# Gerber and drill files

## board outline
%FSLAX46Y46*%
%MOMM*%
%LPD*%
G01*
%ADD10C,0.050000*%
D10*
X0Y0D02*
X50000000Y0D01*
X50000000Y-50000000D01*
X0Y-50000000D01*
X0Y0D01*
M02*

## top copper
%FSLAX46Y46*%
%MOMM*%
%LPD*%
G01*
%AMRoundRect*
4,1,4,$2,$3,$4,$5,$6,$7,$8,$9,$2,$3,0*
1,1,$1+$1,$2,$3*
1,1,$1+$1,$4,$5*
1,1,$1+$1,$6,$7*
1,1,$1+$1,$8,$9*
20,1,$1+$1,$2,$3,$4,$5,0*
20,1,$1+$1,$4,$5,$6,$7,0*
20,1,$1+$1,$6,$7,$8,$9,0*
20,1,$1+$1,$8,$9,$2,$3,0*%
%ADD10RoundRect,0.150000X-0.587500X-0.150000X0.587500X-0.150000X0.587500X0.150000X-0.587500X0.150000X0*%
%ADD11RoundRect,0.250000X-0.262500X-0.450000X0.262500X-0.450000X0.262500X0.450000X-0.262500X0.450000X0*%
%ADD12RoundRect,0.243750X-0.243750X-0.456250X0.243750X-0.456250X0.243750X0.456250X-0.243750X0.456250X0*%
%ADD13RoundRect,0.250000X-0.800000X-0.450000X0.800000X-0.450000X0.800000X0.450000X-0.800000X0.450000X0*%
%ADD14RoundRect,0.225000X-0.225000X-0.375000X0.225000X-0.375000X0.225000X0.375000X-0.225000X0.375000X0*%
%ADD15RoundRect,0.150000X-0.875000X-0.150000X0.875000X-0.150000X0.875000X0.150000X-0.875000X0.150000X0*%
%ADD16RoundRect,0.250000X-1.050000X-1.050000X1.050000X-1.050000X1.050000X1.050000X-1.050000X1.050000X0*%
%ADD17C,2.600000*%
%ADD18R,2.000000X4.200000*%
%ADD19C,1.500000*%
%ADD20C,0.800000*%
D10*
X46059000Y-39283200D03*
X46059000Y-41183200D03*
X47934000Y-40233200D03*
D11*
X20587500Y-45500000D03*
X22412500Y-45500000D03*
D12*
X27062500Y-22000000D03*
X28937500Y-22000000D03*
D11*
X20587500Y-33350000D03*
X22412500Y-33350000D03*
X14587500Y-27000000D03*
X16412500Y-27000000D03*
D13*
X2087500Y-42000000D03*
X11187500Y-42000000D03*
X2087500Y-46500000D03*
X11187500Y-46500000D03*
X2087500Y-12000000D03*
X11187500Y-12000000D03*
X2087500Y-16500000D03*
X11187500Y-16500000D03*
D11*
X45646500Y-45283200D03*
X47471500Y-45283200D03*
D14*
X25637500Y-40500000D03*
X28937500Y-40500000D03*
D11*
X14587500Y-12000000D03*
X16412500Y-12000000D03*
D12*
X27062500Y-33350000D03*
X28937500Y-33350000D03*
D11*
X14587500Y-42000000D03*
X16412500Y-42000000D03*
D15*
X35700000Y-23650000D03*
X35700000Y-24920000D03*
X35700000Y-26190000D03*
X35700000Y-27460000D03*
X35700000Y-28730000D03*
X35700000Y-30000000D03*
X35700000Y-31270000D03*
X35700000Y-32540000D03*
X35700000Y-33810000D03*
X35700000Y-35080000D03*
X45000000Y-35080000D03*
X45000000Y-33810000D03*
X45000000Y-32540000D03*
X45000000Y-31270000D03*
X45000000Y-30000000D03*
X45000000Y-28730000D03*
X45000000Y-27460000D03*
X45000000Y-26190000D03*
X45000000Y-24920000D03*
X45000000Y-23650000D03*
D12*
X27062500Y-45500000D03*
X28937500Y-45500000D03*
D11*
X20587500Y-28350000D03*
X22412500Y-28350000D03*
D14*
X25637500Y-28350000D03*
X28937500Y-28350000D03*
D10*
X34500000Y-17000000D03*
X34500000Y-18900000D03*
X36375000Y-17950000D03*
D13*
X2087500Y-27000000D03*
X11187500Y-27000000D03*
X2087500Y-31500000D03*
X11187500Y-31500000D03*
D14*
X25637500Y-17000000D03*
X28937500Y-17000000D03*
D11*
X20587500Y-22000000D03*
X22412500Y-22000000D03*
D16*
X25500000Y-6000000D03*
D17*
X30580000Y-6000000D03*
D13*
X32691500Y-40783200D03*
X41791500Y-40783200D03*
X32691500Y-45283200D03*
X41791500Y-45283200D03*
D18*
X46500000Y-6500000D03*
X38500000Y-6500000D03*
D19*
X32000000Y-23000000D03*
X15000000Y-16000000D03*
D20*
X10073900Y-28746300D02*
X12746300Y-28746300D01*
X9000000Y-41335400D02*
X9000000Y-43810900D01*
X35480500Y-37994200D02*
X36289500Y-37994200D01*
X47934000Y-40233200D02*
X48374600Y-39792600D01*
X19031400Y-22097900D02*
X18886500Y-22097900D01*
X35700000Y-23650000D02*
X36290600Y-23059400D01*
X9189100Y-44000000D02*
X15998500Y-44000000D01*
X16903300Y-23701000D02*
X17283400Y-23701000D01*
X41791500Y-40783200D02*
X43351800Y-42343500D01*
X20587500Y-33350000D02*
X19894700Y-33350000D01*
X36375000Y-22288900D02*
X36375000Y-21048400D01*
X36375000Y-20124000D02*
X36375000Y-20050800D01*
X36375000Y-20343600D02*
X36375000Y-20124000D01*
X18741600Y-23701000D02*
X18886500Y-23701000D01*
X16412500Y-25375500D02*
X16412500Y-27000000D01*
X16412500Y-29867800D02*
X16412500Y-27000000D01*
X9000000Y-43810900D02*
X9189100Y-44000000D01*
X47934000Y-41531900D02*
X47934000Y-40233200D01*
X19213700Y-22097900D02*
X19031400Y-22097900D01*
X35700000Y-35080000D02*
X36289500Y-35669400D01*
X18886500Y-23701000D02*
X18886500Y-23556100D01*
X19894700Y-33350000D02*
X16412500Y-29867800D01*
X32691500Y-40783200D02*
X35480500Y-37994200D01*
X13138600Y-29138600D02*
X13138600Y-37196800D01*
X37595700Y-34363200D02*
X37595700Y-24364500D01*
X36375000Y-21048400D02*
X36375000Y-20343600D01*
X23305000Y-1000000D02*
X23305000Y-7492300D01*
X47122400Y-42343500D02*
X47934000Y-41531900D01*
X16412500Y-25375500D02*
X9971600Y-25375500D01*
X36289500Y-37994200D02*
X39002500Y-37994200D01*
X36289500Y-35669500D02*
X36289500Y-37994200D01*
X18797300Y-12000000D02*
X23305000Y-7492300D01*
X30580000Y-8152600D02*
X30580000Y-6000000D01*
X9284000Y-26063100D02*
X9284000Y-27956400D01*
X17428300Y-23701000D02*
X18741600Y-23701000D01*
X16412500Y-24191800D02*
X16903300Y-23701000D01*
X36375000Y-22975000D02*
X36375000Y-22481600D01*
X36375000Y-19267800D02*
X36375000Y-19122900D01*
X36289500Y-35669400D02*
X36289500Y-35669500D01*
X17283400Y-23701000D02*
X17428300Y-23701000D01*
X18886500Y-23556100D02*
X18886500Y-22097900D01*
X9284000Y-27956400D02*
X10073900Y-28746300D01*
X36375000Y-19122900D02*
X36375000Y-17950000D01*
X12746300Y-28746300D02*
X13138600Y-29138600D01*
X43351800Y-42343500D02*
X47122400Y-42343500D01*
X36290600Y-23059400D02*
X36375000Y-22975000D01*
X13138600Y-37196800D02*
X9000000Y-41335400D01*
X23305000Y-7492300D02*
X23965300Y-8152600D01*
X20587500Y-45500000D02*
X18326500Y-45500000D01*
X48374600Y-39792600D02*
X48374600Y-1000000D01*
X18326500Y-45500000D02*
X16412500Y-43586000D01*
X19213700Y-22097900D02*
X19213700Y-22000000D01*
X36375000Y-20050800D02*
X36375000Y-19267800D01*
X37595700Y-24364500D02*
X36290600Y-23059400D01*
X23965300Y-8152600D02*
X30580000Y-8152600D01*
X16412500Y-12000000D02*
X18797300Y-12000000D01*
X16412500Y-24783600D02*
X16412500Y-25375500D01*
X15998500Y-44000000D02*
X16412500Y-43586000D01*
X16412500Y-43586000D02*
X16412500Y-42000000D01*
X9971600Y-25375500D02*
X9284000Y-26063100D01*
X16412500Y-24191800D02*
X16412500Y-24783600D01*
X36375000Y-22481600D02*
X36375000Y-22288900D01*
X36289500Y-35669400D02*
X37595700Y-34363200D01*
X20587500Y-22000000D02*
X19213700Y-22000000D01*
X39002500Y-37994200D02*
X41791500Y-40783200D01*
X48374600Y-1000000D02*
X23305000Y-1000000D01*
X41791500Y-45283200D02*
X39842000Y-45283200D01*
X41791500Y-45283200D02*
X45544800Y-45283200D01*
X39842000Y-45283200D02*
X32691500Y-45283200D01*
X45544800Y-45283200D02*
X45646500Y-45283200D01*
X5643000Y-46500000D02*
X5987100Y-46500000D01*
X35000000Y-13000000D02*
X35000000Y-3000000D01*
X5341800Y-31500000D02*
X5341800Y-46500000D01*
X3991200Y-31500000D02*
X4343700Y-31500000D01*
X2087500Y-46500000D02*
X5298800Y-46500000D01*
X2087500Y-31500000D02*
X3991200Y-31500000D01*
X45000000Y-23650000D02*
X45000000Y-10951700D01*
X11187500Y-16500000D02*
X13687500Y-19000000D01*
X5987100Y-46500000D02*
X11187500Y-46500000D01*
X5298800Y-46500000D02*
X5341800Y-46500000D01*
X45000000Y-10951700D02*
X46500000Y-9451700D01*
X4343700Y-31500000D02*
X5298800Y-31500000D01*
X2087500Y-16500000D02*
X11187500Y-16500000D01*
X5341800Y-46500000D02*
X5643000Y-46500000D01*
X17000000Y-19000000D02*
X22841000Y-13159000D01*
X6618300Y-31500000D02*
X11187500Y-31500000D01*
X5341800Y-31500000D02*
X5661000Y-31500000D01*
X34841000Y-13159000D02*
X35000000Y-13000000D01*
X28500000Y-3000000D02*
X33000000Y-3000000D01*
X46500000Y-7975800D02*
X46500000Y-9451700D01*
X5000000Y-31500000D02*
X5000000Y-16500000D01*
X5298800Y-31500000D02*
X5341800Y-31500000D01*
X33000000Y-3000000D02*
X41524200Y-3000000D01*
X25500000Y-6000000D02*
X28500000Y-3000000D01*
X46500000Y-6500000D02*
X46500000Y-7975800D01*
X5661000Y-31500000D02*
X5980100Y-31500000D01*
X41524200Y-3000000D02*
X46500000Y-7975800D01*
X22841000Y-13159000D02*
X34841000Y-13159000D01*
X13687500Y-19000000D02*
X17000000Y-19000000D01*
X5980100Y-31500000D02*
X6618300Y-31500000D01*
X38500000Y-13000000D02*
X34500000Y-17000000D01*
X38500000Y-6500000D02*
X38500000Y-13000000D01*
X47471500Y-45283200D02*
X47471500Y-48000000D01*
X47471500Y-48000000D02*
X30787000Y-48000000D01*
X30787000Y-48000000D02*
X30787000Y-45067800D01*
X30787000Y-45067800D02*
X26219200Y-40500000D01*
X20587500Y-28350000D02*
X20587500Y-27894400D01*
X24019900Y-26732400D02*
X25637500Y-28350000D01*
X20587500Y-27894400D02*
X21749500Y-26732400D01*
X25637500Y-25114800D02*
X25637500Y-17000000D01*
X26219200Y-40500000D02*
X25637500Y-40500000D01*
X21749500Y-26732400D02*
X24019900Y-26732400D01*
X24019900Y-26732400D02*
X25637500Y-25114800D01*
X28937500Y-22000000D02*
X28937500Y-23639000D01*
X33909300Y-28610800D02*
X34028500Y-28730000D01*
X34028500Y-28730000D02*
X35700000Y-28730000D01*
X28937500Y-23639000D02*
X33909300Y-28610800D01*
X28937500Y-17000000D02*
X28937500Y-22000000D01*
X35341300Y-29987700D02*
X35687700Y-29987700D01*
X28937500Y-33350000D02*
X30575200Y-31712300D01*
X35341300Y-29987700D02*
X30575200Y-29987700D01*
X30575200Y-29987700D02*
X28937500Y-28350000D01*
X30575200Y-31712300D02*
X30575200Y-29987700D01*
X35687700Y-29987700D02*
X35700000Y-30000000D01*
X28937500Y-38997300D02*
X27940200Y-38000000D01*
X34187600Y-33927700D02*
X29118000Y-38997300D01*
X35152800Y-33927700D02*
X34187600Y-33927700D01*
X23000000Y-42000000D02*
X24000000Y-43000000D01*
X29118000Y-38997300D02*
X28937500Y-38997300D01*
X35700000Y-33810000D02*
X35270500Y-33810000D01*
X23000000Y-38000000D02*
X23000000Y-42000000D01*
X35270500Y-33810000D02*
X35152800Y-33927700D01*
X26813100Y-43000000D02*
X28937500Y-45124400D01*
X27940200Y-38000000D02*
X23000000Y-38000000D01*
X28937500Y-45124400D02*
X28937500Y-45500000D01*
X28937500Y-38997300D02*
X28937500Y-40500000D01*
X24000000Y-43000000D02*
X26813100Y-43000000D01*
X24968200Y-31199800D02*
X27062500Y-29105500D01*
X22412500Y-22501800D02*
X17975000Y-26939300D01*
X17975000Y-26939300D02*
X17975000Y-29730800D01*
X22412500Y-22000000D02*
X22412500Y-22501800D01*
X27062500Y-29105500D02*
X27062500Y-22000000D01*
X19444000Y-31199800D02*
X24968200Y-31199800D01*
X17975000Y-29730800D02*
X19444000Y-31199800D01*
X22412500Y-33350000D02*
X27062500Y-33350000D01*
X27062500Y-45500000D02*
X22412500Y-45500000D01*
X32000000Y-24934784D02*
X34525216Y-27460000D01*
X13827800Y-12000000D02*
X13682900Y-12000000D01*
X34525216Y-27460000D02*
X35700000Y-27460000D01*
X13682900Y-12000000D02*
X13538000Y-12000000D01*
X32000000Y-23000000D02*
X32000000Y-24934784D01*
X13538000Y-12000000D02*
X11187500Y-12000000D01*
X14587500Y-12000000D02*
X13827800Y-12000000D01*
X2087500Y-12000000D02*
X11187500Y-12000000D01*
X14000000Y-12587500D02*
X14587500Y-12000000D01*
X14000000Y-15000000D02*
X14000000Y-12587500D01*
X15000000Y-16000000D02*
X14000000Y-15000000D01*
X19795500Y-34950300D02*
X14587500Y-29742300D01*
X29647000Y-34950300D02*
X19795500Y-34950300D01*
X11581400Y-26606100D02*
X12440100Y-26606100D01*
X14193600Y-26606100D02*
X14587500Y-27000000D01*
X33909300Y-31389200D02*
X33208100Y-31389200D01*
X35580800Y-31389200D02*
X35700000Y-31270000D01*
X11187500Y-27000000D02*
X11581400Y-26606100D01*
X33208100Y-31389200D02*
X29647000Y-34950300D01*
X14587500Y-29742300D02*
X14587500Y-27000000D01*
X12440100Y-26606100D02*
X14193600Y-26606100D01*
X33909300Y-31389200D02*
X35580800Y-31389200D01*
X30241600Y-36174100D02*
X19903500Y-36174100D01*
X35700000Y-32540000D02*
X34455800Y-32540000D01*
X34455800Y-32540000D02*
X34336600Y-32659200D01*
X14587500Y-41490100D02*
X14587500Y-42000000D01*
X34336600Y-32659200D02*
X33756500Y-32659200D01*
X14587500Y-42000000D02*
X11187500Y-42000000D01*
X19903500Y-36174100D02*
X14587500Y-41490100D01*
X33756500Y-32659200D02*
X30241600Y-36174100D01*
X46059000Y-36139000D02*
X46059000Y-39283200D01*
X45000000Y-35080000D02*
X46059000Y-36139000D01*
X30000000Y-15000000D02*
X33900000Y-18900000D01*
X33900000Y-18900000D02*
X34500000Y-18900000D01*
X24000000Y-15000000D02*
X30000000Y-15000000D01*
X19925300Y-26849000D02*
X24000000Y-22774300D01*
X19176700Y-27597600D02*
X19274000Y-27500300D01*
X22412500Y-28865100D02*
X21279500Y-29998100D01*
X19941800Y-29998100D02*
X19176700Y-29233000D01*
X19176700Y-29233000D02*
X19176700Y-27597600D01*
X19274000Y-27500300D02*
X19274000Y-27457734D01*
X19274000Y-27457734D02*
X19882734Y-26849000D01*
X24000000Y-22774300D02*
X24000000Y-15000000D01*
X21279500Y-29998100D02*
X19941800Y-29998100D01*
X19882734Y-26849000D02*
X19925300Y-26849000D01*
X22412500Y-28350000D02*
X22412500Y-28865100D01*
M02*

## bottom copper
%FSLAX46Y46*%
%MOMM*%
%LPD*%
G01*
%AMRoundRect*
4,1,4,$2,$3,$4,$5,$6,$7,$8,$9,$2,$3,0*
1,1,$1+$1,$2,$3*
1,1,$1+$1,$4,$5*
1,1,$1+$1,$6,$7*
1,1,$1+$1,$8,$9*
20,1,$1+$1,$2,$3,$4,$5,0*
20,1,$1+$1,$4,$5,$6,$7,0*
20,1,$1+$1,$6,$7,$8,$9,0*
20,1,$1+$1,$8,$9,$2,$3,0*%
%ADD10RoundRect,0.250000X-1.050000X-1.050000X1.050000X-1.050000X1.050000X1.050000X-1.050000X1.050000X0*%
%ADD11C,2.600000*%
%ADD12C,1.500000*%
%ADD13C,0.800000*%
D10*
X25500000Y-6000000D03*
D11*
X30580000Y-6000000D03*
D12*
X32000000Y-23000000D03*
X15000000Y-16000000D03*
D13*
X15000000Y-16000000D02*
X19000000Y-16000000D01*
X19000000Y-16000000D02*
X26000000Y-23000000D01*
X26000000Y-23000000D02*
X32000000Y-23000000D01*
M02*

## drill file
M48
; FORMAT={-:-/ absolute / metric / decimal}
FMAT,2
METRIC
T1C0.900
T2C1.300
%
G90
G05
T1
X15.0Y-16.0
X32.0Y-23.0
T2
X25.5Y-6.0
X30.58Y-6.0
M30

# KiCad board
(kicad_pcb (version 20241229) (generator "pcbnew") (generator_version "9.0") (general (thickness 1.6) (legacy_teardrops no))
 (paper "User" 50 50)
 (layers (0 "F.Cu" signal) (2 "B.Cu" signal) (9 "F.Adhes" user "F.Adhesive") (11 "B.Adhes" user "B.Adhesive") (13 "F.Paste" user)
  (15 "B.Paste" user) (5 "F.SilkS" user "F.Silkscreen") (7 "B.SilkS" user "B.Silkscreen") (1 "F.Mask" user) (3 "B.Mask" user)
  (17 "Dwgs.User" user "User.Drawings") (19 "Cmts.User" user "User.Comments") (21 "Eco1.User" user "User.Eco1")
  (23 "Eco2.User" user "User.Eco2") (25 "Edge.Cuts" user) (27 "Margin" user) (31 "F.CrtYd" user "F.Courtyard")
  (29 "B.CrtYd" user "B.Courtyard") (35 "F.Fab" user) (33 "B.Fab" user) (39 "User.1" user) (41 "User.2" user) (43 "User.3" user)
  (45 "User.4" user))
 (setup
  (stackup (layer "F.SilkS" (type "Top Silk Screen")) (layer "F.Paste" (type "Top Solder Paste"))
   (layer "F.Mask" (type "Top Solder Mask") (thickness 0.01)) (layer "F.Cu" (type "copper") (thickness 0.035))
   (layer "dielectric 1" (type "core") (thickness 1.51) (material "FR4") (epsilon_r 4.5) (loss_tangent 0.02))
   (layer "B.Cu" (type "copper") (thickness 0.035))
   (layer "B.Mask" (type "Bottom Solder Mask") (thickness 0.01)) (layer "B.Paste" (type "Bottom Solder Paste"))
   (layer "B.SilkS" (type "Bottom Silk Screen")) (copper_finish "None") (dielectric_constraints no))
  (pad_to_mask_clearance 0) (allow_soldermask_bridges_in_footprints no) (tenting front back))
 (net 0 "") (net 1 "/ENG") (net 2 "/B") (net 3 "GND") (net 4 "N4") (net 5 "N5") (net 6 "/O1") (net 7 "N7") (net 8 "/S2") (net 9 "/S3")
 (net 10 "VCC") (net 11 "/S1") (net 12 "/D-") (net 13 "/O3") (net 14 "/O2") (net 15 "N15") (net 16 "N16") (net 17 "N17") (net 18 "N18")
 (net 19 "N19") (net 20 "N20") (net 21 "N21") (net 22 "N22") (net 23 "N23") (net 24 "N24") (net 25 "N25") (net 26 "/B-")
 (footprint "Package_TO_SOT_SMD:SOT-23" (layer "F.Cu") (at 46.9965 40.2332)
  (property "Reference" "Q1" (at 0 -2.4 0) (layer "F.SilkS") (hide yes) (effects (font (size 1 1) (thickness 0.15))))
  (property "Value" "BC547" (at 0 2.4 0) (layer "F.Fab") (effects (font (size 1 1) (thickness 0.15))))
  (pad "1" smd roundrect (at -0.9375 -0.95) (size 1.475 0.6) (layers "F.Cu" "F.Mask" "F.Paste") (roundrect_rratio 0.25) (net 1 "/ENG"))
  (pad "2" smd roundrect (at -0.9375 0.95) (size 1.475 0.6) (layers "F.Cu" "F.Mask" "F.Paste") (roundrect_rratio 0.25) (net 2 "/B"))
  (pad "3" smd roundrect (at 0.9375 0) (size 1.475 0.6) (layers "F.Cu" "F.Mask" "F.Paste") (roundrect_rratio 0.25) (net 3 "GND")))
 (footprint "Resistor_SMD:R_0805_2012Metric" (layer "F.Cu") (at 21.5 45.5)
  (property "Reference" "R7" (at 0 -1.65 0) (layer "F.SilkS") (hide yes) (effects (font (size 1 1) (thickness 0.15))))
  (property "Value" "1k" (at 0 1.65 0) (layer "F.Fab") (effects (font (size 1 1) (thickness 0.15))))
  (pad "1" smd roundrect (at -0.9125 0) (size 1.025 1.4) (layers "F.Cu" "F.Mask" "F.Paste") (roundrect_rratio 0.243902) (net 3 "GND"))
  (pad "2" smd roundrect (at 0.9125 0) (size 1.025 1.4) (layers "F.Cu" "F.Mask" "F.Paste") (roundrect_rratio 0.243902) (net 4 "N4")))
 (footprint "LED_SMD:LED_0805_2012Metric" (layer "F.Cu") (at 28 22)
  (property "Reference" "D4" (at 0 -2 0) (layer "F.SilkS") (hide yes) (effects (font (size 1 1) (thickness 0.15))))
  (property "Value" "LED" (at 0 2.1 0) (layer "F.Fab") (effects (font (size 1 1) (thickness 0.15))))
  (pad "1" smd roundrect (at -0.9375 0) (size 0.975 1.4) (layers "F.Cu" "F.Mask" "F.Paste") (roundrect_rratio 0.25) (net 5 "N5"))
  (pad "2" smd roundrect (at 0.9375 0) (size 0.975 1.4) (layers "F.Cu" "F.Mask" "F.Paste") (roundrect_rratio 0.25) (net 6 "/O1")))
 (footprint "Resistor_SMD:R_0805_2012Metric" (layer "F.Cu") (at 21.5 33.35)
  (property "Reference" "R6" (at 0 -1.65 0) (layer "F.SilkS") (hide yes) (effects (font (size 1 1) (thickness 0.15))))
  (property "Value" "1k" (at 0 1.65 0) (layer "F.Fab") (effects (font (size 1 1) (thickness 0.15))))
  (pad "1" smd roundrect (at -0.9125 0) (size 1.025 1.4) (layers "F.Cu" "F.Mask" "F.Paste") (roundrect_rratio 0.243902) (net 3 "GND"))
  (pad "2" smd roundrect (at 0.9125 0) (size 1.025 1.4) (layers "F.Cu" "F.Mask" "F.Paste") (roundrect_rratio 0.243902) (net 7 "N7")))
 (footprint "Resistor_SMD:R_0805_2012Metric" (layer "F.Cu") (at 15.5 27)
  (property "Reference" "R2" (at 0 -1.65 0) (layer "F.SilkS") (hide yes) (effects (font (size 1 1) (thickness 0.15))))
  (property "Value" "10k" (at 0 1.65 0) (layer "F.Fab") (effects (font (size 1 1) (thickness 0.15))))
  (pad "1" smd roundrect (at -0.9125 0) (size 1.025 1.4) (layers "F.Cu" "F.Mask" "F.Paste") (roundrect_rratio 0.243902) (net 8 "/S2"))
  (pad "2" smd roundrect (at 0.9125 0) (size 1.025 1.4) (layers "F.Cu" "F.Mask" "F.Paste") (roundrect_rratio 0.243902) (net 3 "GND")))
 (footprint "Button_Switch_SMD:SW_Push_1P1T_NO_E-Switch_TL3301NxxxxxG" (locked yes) (layer "F.Cu") (at 6.6375 44.25)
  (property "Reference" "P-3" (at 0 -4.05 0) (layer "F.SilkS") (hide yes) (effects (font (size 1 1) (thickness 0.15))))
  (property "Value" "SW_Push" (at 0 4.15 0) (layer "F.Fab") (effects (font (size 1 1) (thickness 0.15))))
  (pad "1" smd roundrect (at -4.55 -2.25) (size 2.1 1.4) (layers "F.Cu" "F.Mask" "F.Paste") (roundrect_rratio 0.1785714286) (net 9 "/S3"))
  (pad "1" smd roundrect (at 4.55 -2.25) (size 2.1 1.4) (layers "F.Cu" "F.Mask" "F.Paste") (roundrect_rratio 0.1785714286) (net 9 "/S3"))
  (pad "2" smd roundrect (at -4.55 2.25) (size 2.1 1.4) (layers "F.Cu" "F.Mask" "F.Paste") (roundrect_rratio 0.1785714286) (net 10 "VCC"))
  (pad "2" smd roundrect (at 4.55 2.25) (size 2.1 1.4) (layers "F.Cu" "F.Mask" "F.Paste") (roundrect_rratio 0.1785714286) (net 10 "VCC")))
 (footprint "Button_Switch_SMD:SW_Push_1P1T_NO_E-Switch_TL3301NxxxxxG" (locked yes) (layer "F.Cu") (at 6.6375 14.25)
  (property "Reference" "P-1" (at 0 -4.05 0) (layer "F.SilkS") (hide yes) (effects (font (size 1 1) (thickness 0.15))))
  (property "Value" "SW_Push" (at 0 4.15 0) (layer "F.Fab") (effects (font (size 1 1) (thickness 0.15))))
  (pad "1" smd roundrect (at -4.55 -2.25) (size 2.1 1.4) (layers "F.Cu" "F.Mask" "F.Paste") (roundrect_rratio 0.1785714286) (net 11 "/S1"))
  (pad "1" smd roundrect (at 4.55 -2.25) (size 2.1 1.4) (layers "F.Cu" "F.Mask" "F.Paste") (roundrect_rratio 0.1785714286) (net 11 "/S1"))
  (pad "2" smd roundrect (at -4.55 2.25) (size 2.1 1.4) (layers "F.Cu" "F.Mask" "F.Paste") (roundrect_rratio 0.1785714286) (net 10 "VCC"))
  (pad "2" smd roundrect (at 4.55 2.25) (size 2.1 1.4) (layers "F.Cu" "F.Mask" "F.Paste") (roundrect_rratio 0.1785714286) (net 10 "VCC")))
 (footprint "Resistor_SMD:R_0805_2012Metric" (layer "F.Cu") (at 46.559 45.2832)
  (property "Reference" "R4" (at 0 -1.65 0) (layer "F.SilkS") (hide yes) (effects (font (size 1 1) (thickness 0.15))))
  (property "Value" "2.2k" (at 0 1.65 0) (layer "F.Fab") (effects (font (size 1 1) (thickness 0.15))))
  (pad "1" smd roundrect (at -0.9125 0) (size 1.025 1.4) (layers "F.Cu" "F.Mask" "F.Paste") (roundrect_rratio 0.243902) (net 2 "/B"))
  (pad "2" smd roundrect (at 0.9125 0) (size 1.025 1.4) (layers "F.Cu" "F.Mask" "F.Paste") (roundrect_rratio 0.243902) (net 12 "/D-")))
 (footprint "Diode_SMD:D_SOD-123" (layer "F.Cu") (at 27.2875 40.5)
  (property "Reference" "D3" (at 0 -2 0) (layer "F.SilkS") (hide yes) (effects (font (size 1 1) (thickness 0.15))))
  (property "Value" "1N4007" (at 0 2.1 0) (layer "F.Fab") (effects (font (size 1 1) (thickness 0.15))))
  (pad "1" smd roundrect (at -1.65 0) (size 0.9 1.2) (layers "F.Cu" "F.Mask" "F.Paste") (roundrect_rratio 0.25) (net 12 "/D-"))
  (pad "2" smd roundrect (at 1.65 0) (size 0.9 1.2) (layers "F.Cu" "F.Mask" "F.Paste") (roundrect_rratio 0.25) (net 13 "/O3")))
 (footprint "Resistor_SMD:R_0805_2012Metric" (layer "F.Cu") (at 15.5 12)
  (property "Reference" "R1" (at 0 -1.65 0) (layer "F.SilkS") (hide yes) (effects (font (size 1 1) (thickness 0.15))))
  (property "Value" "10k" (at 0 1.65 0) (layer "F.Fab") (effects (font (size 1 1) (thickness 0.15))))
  (pad "1" smd roundrect (at -0.9125 0) (size 1.025 1.4) (layers "F.Cu" "F.Mask" "F.Paste") (roundrect_rratio 0.243902) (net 11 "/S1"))
  (pad "2" smd roundrect (at 0.9125 0) (size 1.025 1.4) (layers "F.Cu" "F.Mask" "F.Paste") (roundrect_rratio 0.243902) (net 3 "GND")))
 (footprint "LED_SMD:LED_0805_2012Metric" (layer "F.Cu") (at 28 33.35)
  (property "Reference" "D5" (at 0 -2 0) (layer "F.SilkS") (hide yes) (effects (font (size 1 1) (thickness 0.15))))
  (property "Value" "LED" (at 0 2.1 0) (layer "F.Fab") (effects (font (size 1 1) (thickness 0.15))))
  (pad "1" smd roundrect (at -0.9375 0) (size 0.975 1.4) (layers "F.Cu" "F.Mask" "F.Paste") (roundrect_rratio 0.25) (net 7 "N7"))
  (pad "2" smd roundrect (at 0.9375 0) (size 0.975 1.4) (layers "F.Cu" "F.Mask" "F.Paste") (roundrect_rratio 0.25) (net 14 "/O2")))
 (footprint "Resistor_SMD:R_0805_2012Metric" (layer "F.Cu") (at 15.5 42)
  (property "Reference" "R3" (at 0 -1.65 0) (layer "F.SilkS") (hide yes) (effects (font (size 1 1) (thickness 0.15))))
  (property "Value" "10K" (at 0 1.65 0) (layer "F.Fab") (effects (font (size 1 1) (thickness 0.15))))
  (pad "1" smd roundrect (at -0.9125 0) (size 1.025 1.4) (layers "F.Cu" "F.Mask" "F.Paste") (roundrect_rratio 0.243902) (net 9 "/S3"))
  (pad "2" smd roundrect (at 0.9125 0) (size 1.025 1.4) (layers "F.Cu" "F.Mask" "F.Paste") (roundrect_rratio 0.243902) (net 3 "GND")))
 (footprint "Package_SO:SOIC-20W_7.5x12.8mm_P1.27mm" (layer "F.Cu") (at 40.35 29.365)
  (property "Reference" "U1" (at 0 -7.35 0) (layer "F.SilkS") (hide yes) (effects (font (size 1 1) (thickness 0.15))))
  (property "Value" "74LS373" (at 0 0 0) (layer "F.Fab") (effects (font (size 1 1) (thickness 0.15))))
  (pad "1" smd roundrect (at -4.65 -5.715) (size 2.05 0.6) (layers "F.Cu" "F.Mask" "F.Paste") (roundrect_rratio 0.25) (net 3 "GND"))
  (pad "2" smd roundrect (at -4.65 -4.445) (size 2.05 0.6) (layers "F.Cu" "F.Mask" "F.Paste") (roundrect_rratio 0.25) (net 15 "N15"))
  (pad "3" smd roundrect (at -4.65 -3.175) (size 2.05 0.6) (layers "F.Cu" "F.Mask" "F.Paste") (roundrect_rratio 0.25) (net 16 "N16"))
  (pad "4" smd roundrect (at -4.65 -1.905) (size 2.05 0.6) (layers "F.Cu" "F.Mask" "F.Paste") (roundrect_rratio 0.25) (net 11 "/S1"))
  (pad "5" smd roundrect (at -4.65 -0.635) (size 2.05 0.6) (layers "F.Cu" "F.Mask" "F.Paste") (roundrect_rratio 0.25) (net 6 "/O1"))
  (pad "6" smd roundrect (at -4.65 0.635) (size 2.05 0.6) (layers "F.Cu" "F.Mask" "F.Paste") (roundrect_rratio 0.25) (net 14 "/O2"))
  (pad "7" smd roundrect (at -4.65 1.905) (size 2.05 0.6) (layers "F.Cu" "F.Mask" "F.Paste") (roundrect_rratio 0.25) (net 8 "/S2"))
  (pad "8" smd roundrect (at -4.65 3.175) (size 2.05 0.6) (layers "F.Cu" "F.Mask" "F.Paste") (roundrect_rratio 0.25) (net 9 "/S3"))
  (pad "9" smd roundrect (at -4.65 4.445) (size 2.05 0.6) (layers "F.Cu" "F.Mask" "F.Paste") (roundrect_rratio 0.25) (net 13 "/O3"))
  (pad "10" smd roundrect (at -4.65 5.715) (size 2.05 0.6) (layers "F.Cu" "F.Mask" "F.Paste") (roundrect_rratio 0.25) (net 3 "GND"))
  (pad "11" smd roundrect (at 4.65 5.715) (size 2.05 0.6) (layers "F.Cu" "F.Mask" "F.Paste") (roundrect_rratio 0.25) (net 1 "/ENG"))
  (pad "12" smd roundrect (at 4.65 4.445) (size 2.05 0.6) (layers "F.Cu" "F.Mask" "F.Paste") (roundrect_rratio 0.25) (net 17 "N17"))
  (pad "13" smd roundrect (at 4.65 3.175) (size 2.05 0.6) (layers "F.Cu" "F.Mask" "F.Paste") (roundrect_rratio 0.25) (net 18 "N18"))
  (pad "14" smd roundrect (at 4.65 1.905) (size 2.05 0.6) (layers "F.Cu" "F.Mask" "F.Paste") (roundrect_rratio 0.25) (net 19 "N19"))
  (pad "15" smd roundrect (at 4.65 0.635) (size 2.05 0.6) (layers "F.Cu" "F.Mask" "F.Paste") (roundrect_rratio 0.25) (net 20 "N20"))
  (pad "16" smd roundrect (at 4.65 -0.635) (size 2.05 0.6) (layers "F.Cu" "F.Mask" "F.Paste") (roundrect_rratio 0.25) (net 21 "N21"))
  (pad "17" smd roundrect (at 4.65 -1.905) (size 2.05 0.6) (layers "F.Cu" "F.Mask" "F.Paste") (roundrect_rratio 0.25) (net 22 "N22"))
  (pad "18" smd roundrect (at 4.65 -3.175) (size 2.05 0.6) (layers "F.Cu" "F.Mask" "F.Paste") (roundrect_rratio 0.25) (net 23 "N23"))
  (pad "19" smd roundrect (at 4.65 -4.445) (size 2.05 0.6) (layers "F.Cu" "F.Mask" "F.Paste") (roundrect_rratio 0.25) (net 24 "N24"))
  (pad "20" smd roundrect (at 4.65 -5.715) (size 2.05 0.6) (layers "F.Cu" "F.Mask" "F.Paste") (roundrect_rratio 0.25) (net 10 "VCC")))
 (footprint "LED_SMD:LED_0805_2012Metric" (layer "F.Cu") (at 28 45.5)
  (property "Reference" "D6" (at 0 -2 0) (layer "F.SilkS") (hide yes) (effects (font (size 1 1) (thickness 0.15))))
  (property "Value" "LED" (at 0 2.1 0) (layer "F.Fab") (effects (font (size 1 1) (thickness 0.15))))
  (pad "1" smd roundrect (at -0.9375 0) (size 0.975 1.4) (layers "F.Cu" "F.Mask" "F.Paste") (roundrect_rratio 0.25) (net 4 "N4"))
  (pad "2" smd roundrect (at 0.9375 0) (size 0.975 1.4) (layers "F.Cu" "F.Mask" "F.Paste") (roundrect_rratio 0.25) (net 13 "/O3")))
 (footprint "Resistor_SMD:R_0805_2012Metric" (layer "F.Cu") (at 21.5 28.35)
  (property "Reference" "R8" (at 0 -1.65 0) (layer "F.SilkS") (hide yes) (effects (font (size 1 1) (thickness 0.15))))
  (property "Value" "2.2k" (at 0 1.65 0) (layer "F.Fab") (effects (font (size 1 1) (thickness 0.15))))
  (pad "1" smd roundrect (at -0.9125 0) (size 1.025 1.4) (layers "F.Cu" "F.Mask" "F.Paste") (roundrect_rratio 0.243902) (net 12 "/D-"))
  (pad "2" smd roundrect (at 0.9125 0) (size 1.025 1.4) (layers "F.Cu" "F.Mask" "F.Paste") (roundrect_rratio 0.243902) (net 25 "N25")))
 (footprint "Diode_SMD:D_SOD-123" (layer "F.Cu") (at 27.2875 28.35)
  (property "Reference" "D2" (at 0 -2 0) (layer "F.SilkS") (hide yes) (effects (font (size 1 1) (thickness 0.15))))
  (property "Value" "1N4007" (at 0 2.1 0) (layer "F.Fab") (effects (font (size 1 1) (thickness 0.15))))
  (pad "1" smd roundrect (at -1.65 0) (size 0.9 1.2) (layers "F.Cu" "F.Mask" "F.Paste") (roundrect_rratio 0.25) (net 12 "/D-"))
  (pad "2" smd roundrect (at 1.65 0) (size 0.9 1.2) (layers "F.Cu" "F.Mask" "F.Paste") (roundrect_rratio 0.25) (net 14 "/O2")))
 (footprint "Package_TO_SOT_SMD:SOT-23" (layer "F.Cu") (at 35.4375 17.95)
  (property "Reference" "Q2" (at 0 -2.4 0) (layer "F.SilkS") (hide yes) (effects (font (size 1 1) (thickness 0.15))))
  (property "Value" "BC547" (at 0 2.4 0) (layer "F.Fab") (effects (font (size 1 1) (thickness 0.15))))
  (pad "1" smd roundrect (at -0.9375 -0.95) (size 1.475 0.6) (layers "F.Cu" "F.Mask" "F.Paste") (roundrect_rratio 0.25) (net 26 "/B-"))
  (pad "2" smd roundrect (at -0.9375 0.95) (size 1.475 0.6) (layers "F.Cu" "F.Mask" "F.Paste") (roundrect_rratio 0.25) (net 25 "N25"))
  (pad "3" smd roundrect (at 0.9375 0) (size 1.475 0.6) (layers "F.Cu" "F.Mask" "F.Paste") (roundrect_rratio 0.25) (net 3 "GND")))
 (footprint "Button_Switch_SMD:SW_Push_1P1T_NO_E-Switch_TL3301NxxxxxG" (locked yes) (layer "F.Cu") (at 6.6375 29.25)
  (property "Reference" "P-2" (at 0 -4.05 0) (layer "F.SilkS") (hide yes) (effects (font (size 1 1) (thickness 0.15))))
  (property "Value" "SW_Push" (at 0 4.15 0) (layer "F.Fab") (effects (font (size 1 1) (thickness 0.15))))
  (pad "1" smd roundrect (at -4.55 -2.25) (size 2.1 1.4) (layers "F.Cu" "F.Mask" "F.Paste") (roundrect_rratio 0.1785714286) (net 8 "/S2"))
  (pad "1" smd roundrect (at 4.55 -2.25) (size 2.1 1.4) (layers "F.Cu" "F.Mask" "F.Paste") (roundrect_rratio 0.1785714286) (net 8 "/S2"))
  (pad "2" smd roundrect (at -4.55 2.25) (size 2.1 1.4) (layers "F.Cu" "F.Mask" "F.Paste") (roundrect_rratio 0.1785714286) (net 10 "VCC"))
  (pad "2" smd roundrect (at 4.55 2.25) (size 2.1 1.4) (layers "F.Cu" "F.Mask" "F.Paste") (roundrect_rratio 0.1785714286) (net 10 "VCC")))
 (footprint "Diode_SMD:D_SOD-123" (layer "F.Cu") (at 27.2875 17)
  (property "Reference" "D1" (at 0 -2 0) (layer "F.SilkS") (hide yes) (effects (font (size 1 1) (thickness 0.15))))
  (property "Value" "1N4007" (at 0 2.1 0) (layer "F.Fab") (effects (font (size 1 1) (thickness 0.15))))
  (pad "1" smd roundrect (at -1.65 0) (size 0.9 1.2) (layers "F.Cu" "F.Mask" "F.Paste") (roundrect_rratio 0.25) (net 12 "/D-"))
  (pad "2" smd roundrect (at 1.65 0) (size 0.9 1.2) (layers "F.Cu" "F.Mask" "F.Paste") (roundrect_rratio 0.25) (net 6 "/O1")))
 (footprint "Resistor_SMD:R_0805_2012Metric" (layer "F.Cu") (at 21.5 22)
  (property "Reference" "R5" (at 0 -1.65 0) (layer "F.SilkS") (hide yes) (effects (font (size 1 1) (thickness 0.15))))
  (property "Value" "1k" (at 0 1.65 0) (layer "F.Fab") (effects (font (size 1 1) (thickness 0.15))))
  (pad "1" smd roundrect (at -0.9125 0) (size 1.025 1.4) (layers "F.Cu" "F.Mask" "F.Paste") (roundrect_rratio 0.243902) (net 3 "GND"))
  (pad "2" smd roundrect (at 0.9125 0) (size 1.025 1.4) (layers "F.Cu" "F.Mask" "F.Paste") (roundrect_rratio 0.243902) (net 5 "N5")))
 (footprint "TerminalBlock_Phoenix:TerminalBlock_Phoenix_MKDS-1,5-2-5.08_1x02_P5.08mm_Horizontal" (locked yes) (layer "F.Cu") (at 25.5 6)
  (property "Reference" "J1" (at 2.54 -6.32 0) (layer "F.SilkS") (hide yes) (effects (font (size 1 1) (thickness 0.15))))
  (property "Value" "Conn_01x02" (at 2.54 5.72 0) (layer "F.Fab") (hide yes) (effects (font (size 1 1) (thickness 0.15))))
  (pad "1" thru_hole roundrect (at 0 0) (size 2.6 2.6) (drill 1.3) (layers "*.Cu" "*.Mask") (remove_unused_layers no)
   (roundrect_rratio 0.096154) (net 10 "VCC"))
  (pad "2" thru_hole circle (at 5.08 0) (size 2.6 2.6) (drill 1.3) (layers "*.Cu" "*.Mask") (remove_unused_layers no) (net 3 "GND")))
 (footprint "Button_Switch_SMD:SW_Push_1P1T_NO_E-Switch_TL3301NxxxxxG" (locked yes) (layer "F.Cu") (at 37.2415 43.0332)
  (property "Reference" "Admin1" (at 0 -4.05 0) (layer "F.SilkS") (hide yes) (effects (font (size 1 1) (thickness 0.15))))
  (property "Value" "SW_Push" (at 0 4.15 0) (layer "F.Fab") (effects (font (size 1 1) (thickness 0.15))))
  (pad "1" smd roundrect (at -4.55 -2.25) (size 2.1 1.4) (layers "F.Cu" "F.Mask" "F.Paste") (roundrect_rratio 0.1785714286) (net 3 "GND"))
  (pad "1" smd roundrect (at 4.55 -2.25) (size 2.1 1.4) (layers "F.Cu" "F.Mask" "F.Paste") (roundrect_rratio 0.1785714286) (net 3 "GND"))
  (pad "2" smd roundrect (at -4.55 2.25) (size 2.1 1.4) (layers "F.Cu" "F.Mask" "F.Paste") (roundrect_rratio 0.1785714286) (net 2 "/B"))
  (pad "2" smd roundrect (at 4.55 2.25) (size 2.1 1.4) (layers "F.Cu" "F.Mask" "F.Paste") (roundrect_rratio 0.1785714286) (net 2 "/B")))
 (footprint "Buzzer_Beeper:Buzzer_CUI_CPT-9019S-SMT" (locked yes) (layer "F.Cu") (at 42.5 6.5 180)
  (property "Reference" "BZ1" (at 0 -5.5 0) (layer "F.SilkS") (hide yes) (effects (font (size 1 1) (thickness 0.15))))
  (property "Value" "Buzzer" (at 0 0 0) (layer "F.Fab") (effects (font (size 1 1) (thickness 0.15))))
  (pad "1" smd rect (at -4 0 180) (size 2 4.2) (layers "F.Cu" "F.Mask" "F.Paste") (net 10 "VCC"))
  (pad "2" smd rect (at 4 0 180) (size 2 4.2) (layers "F.Cu" "F.Mask" "F.Paste") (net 26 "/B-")))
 (gr_rect (start 0 0) (end 50 50) (stroke (width 0.05) (type solid)) (fill no) (locked yes) (layer "Edge.Cuts"))
 (segment (start 10.0739 28.7463) (end 12.7463 28.7463) (width 0.8) (layer "F.Cu") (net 3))
 (segment (start 9 41.3354) (end 9 43.8109) (width 0.8) (layer "F.Cu") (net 3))
 (segment (start 35.4805 37.9942) (end 36.2895 37.9942) (width 0.8) (layer "F.Cu") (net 3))
 (segment (start 47.934 40.2332) (end 48.3746 39.7926) (width 0.8) (layer "F.Cu") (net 3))
 (segment (start 19.0314 22.0979) (end 18.8865 22.0979) (width 0.8) (layer "F.Cu") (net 3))
 (segment (start 35.7 23.65) (end 36.2906 23.0594) (width 0.8) (layer "F.Cu") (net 3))
 (segment (start 9.1891 44) (end 15.9985 44) (width 0.8) (layer "F.Cu") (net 3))
 (segment (start 16.9033 23.701) (end 17.2834 23.701) (width 0.8) (layer "F.Cu") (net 3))
 (segment (start 41.7915 40.7832) (end 43.3518 42.3435) (width 0.8) (layer "F.Cu") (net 3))
 (segment (start 20.5875 33.35) (end 19.8947 33.35) (width 0.8) (layer "F.Cu") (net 3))
 (segment (start 36.375 22.2889) (end 36.375 21.0484) (width 0.8) (layer "F.Cu") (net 3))
 (segment (start 36.375 20.124) (end 36.375 20.0508) (width 0.8) (layer "F.Cu") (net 3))
 (segment (start 36.375 20.3436) (end 36.375 20.124) (width 0.8) (layer "F.Cu") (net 3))
 (segment (start 18.7416 23.701) (end 18.8865 23.701) (width 0.8) (layer "F.Cu") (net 3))
 (segment (start 16.4125 25.3755) (end 16.4125 27) (width 0.8) (layer "F.Cu") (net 3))
 (segment (start 16.4125 29.8678) (end 16.4125 27) (width 0.8) (layer "F.Cu") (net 3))
 (segment (start 9 43.8109) (end 9.1891 44) (width 0.8) (layer "F.Cu") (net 3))
 (segment (start 47.934 41.5319) (end 47.934 40.2332) (width 0.8) (layer "F.Cu") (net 3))
 (segment (start 19.2137 22.0979) (end 19.0314 22.0979) (width 0.8) (layer "F.Cu") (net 3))
 (segment (start 35.7 35.08) (end 36.2895 35.6694) (width 0.8) (layer "F.Cu") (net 3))
 (segment (start 18.8865 23.701) (end 18.8865 23.5561) (width 0.8) (layer "F.Cu") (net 3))
 (segment (start 19.8947 33.35) (end 16.4125 29.8678) (width 0.8) (layer "F.Cu") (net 3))
 (segment (start 32.6915 40.7832) (end 35.4805 37.9942) (width 0.8) (layer "F.Cu") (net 3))
 (segment (start 13.1386 29.1386) (end 13.1386 37.1968) (width 0.8) (layer "F.Cu") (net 3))
 (segment (start 37.5957 34.3632) (end 37.5957 24.3645) (width 0.8) (layer "F.Cu") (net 3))
 (segment (start 36.375 21.0484) (end 36.375 20.3436) (width 0.8) (layer "F.Cu") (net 3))
 (segment (start 23.305 1) (end 23.305 7.4923) (width 0.8) (layer "F.Cu") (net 3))
 (segment (start 47.1224 42.3435) (end 47.934 41.5319) (width 0.8) (layer "F.Cu") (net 3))
 (segment (start 16.4125 25.3755) (end 9.9716 25.3755) (width 0.8) (layer "F.Cu") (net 3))
 (segment (start 36.2895 37.9942) (end 39.0025 37.9942) (width 0.8) (layer "F.Cu") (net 3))
 (segment (start 36.2895 35.6695) (end 36.2895 37.9942) (width 0.8) (layer "F.Cu") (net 3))
 (segment (start 18.7973 12) (end 23.305 7.4923) (width 0.8) (layer "F.Cu") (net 3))
 (segment (start 30.58 8.1526) (end 30.58 6) (width 0.8) (layer "F.Cu") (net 3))
 (segment (start 9.284 26.0631) (end 9.284 27.9564) (width 0.8) (layer "F.Cu") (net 3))
 (segment (start 17.4283 23.701) (end 18.7416 23.701) (width 0.8) (layer "F.Cu") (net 3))
 (segment (start 16.4125 24.1918) (end 16.9033 23.701) (width 0.8) (layer "F.Cu") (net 3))
 (segment (start 36.375 22.975) (end 36.375 22.4816) (width 0.8) (layer "F.Cu") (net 3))
 (segment (start 36.375 19.2678) (end 36.375 19.1229) (width 0.8) (layer "F.Cu") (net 3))
 (segment (start 36.2895 35.6694) (end 36.2895 35.6695) (width 0.8) (layer "F.Cu") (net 3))
 (segment (start 17.2834 23.701) (end 17.4283 23.701) (width 0.8) (layer "F.Cu") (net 3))
 (segment (start 18.8865 23.5561) (end 18.8865 22.0979) (width 0.8) (layer "F.Cu") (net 3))
 (segment (start 9.284 27.9564) (end 10.0739 28.7463) (width 0.8) (layer "F.Cu") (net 3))
 (segment (start 36.375 19.1229) (end 36.375 17.95) (width 0.8) (layer "F.Cu") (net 3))
 (segment (start 12.7463 28.7463) (end 13.1386 29.1386) (width 0.8) (layer "F.Cu") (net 3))
 (segment (start 43.3518 42.3435) (end 47.1224 42.3435) (width 0.8) (layer "F.Cu") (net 3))
 (segment (start 36.2906 23.0594) (end 36.375 22.975) (width 0.8) (layer "F.Cu") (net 3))
 (segment (start 13.1386 37.1968) (end 9 41.3354) (width 0.8) (layer "F.Cu") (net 3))
 (segment (start 23.305 7.4923) (end 23.9653 8.1526) (width 0.8) (layer "F.Cu") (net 3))
 (segment (start 20.5875 45.5) (end 18.3265 45.5) (width 0.8) (layer "F.Cu") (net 3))
 (segment (start 48.3746 39.7926) (end 48.3746 1) (width 0.8) (layer "F.Cu") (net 3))
 (segment (start 18.3265 45.5) (end 16.4125 43.586) (width 0.8) (layer "F.Cu") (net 3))
 (segment (start 19.2137 22.0979) (end 19.2137 22) (width 0.8) (layer "F.Cu") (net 3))
 (segment (start 36.375 20.0508) (end 36.375 19.2678) (width 0.8) (layer "F.Cu") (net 3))
 (segment (start 37.5957 24.3645) (end 36.2906 23.0594) (width 0.8) (layer "F.Cu") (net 3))
 (segment (start 23.9653 8.1526) (end 30.58 8.1526) (width 0.8) (layer "F.Cu") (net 3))
 (segment (start 16.4125 12) (end 18.7973 12) (width 0.8) (layer "F.Cu") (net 3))
 (segment (start 16.4125 24.7836) (end 16.4125 25.3755) (width 0.8) (layer "F.Cu") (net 3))
 (segment (start 15.9985 44) (end 16.4125 43.586) (width 0.8) (layer "F.Cu") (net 3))
 (segment (start 16.4125 43.586) (end 16.4125 42) (width 0.8) (layer "F.Cu") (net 3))
 (segment (start 9.9716 25.3755) (end 9.284 26.0631) (width 0.8) (layer "F.Cu") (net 3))
 (segment (start 16.4125 24.1918) (end 16.4125 24.7836) (width 0.8) (layer "F.Cu") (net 3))
 (segment (start 36.375 22.4816) (end 36.375 22.2889) (width 0.8) (layer "F.Cu") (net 3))
 (segment (start 36.2895 35.6694) (end 37.5957 34.3632) (width 0.8) (layer "F.Cu") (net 3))
 (segment (start 20.5875 22) (end 19.2137 22) (width 0.8) (layer "F.Cu") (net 3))
 (segment (start 39.0025 37.9942) (end 41.7915 40.7832) (width 0.8) (layer "F.Cu") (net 3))
 (segment (start 48.3746 1) (end 23.305 1) (width 0.8) (layer "F.Cu") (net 3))
 (segment (start 41.7915 45.2832) (end 39.842 45.2832) (width 0.8) (layer "F.Cu") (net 2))
 (segment (start 41.7915 45.2832) (end 45.5448 45.2832) (width 0.8) (layer "F.Cu") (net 2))
 (segment (start 39.842 45.2832) (end 32.6915 45.2832) (width 0.8) (layer "F.Cu") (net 2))
 (segment (start 45.5448 45.2832) (end 45.6465 45.2832) (width 0.8) (layer "F.Cu") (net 2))
 (segment (start 5.643 46.5) (end 5.9871 46.5) (width 0.8) (layer "F.Cu") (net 10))
 (segment (start 35 13) (end 35 3) (width 0.8) (layer "F.Cu") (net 10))
 (segment (start 5.3418 31.5) (end 5.3418 46.5) (width 0.8) (layer "F.Cu") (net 10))
 (segment (start 3.9912 31.5) (end 4.3437 31.5) (width 0.8) (layer "F.Cu") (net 10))
 (segment (start 2.0875 46.5) (end 5.2988 46.5) (width 0.8) (layer "F.Cu") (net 10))
 (segment (start 2.0875 31.5) (end 3.9912 31.5) (width 0.8) (layer "F.Cu") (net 10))
 (segment (start 45 23.65) (end 45 10.9517) (width 0.8) (layer "F.Cu") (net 10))
 (segment (start 11.1875 16.5) (end 13.6875 19) (width 0.8) (layer "F.Cu") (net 10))
 (segment (start 5.9871 46.5) (end 11.1875 46.5) (width 0.8) (layer "F.Cu") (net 10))
 (segment (start 5.2988 46.5) (end 5.3418 46.5) (width 0.8) (layer "F.Cu") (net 10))
 (segment (start 45 10.9517) (end 46.5 9.4517) (width 0.8) (layer "F.Cu") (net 10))
 (segment (start 4.3437 31.5) (end 5.2988 31.5) (width 0.8) (layer "F.Cu") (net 10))
 (segment (start 2.0875 16.5) (end 11.1875 16.5) (width 0.8) (layer "F.Cu") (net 10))
 (segment (start 5.3418 46.5) (end 5.643 46.5) (width 0.8) (layer "F.Cu") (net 10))
 (segment (start 17 19) (end 22.841 13.159) (width 0.8) (layer "F.Cu") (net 10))
 (segment (start 6.6183 31.5) (end 11.1875 31.5) (width 0.8) (layer "F.Cu") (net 10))
 (segment (start 5.3418 31.5) (end 5.661 31.5) (width 0.8) (layer "F.Cu") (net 10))
 (segment (start 34.841 13.159) (end 35 13) (width 0.8) (layer "F.Cu") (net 10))
 (segment (start 28.5 3) (end 33 3) (width 0.8) (layer "F.Cu") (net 10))
 (segment (start 46.5 7.9758) (end 46.5 9.4517) (width 0.8) (layer "F.Cu") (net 10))
 (segment (start 5 31.5) (end 5 16.5) (width 0.8) (layer "F.Cu") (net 10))
 (segment (start 5.2988 31.5) (end 5.3418 31.5) (width 0.8) (layer "F.Cu") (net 10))
 (segment (start 33 3) (end 41.5242 3) (width 0.8) (layer "F.Cu") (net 10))
 (segment (start 25.5 6) (end 28.5 3) (width 0.8) (layer "F.Cu") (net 10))
 (segment (start 46.5 6.5) (end 46.5 7.9758) (width 0.8) (layer "F.Cu") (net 10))
 (segment (start 5.661 31.5) (end 5.9801 31.5) (width 0.8) (layer "F.Cu") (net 10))
 (segment (start 41.5242 3) (end 46.5 7.9758) (width 0.8) (layer "F.Cu") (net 10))
 (segment (start 22.841 13.159) (end 34.841 13.159) (width 0.8) (layer "F.Cu") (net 10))
 (segment (start 13.6875 19) (end 17 19) (width 0.8) (layer "F.Cu") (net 10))
 (segment (start 5.9801 31.5) (end 6.6183 31.5) (width 0.8) (layer "F.Cu") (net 10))
 (segment (start 38.5 13) (end 34.5 17) (width 0.8) (layer "F.Cu") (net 26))
 (segment (start 38.5 6.5) (end 38.5 13) (width 0.8) (layer "F.Cu") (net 26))
 (segment (start 47.4715 45.2832) (end 47.4715 48) (width 0.8) (layer "F.Cu") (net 12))
 (segment (start 47.4715 48) (end 30.787 48) (width 0.8) (layer "F.Cu") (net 12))
 (segment (start 30.787 48) (end 30.787 45.0678) (width 0.8) (layer "F.Cu") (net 12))
 (segment (start 30.787 45.0678) (end 26.2192 40.5) (width 0.8) (layer "F.Cu") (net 12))
 (segment (start 20.5875 28.35) (end 20.5875 27.8944) (width 0.8) (layer "F.Cu") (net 12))
 (segment (start 24.0199 26.7324) (end 25.6375 28.35) (width 0.8) (layer "F.Cu") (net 12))
 (segment (start 20.5875 27.8944) (end 21.7495 26.7324) (width 0.8) (layer "F.Cu") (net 12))
 (segment (start 25.6375 25.1148) (end 25.6375 17) (width 0.8) (layer "F.Cu") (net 12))
 (segment (start 26.2192 40.5) (end 25.6375 40.5) (width 0.8) (layer "F.Cu") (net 12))
 (segment (start 21.7495 26.7324) (end 24.0199 26.7324) (width 0.8) (layer "F.Cu") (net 12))
 (segment (start 24.0199 26.7324) (end 25.6375 25.1148) (width 0.8) (layer "F.Cu") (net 12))
 (segment (start 28.9375 22) (end 28.9375 23.639) (width 0.8) (layer "F.Cu") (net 6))
 (segment (start 33.9093 28.6108) (end 34.0285 28.73) (width 0.8) (layer "F.Cu") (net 6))
 (segment (start 34.0285 28.73) (end 35.7 28.73) (width 0.8) (layer "F.Cu") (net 6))
 (segment (start 28.9375 23.639) (end 33.9093 28.6108) (width 0.8) (layer "F.Cu") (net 6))
 (segment (start 28.9375 17) (end 28.9375 22) (width 0.8) (layer "F.Cu") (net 6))
 (segment (start 35.3413 29.9877) (end 35.6877 29.9877) (width 0.8) (layer "F.Cu") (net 14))
 (segment (start 28.9375 33.35) (end 30.5752 31.7123) (width 0.8) (layer "F.Cu") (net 14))
 (segment (start 35.3413 29.9877) (end 30.5752 29.9877) (width 0.8) (layer "F.Cu") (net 14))
 (segment (start 30.5752 29.9877) (end 28.9375 28.35) (width 0.8) (layer "F.Cu") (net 14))
 (segment (start 30.5752 31.7123) (end 30.5752 29.9877) (width 0.8) (layer "F.Cu") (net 14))
 (segment (start 35.6877 29.9877) (end 35.7 30) (width 0.8) (layer "F.Cu") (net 14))
 (segment (start 28.9375 38.9973) (end 27.9402 38) (width 0.8) (layer "F.Cu") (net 13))
 (segment (start 34.1876 33.9277) (end 29.118 38.9973) (width 0.8) (layer "F.Cu") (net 13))
 (segment (start 35.1528 33.9277) (end 34.1876 33.9277) (width 0.8) (layer "F.Cu") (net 13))
 (segment (start 23 42) (end 24 43) (width 0.8) (layer "F.Cu") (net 13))
 (segment (start 29.118 38.9973) (end 28.9375 38.9973) (width 0.8) (layer "F.Cu") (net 13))
 (segment (start 35.7 33.81) (end 35.2705 33.81) (width 0.8) (layer "F.Cu") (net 13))
 (segment (start 23 38) (end 23 42) (width 0.8) (layer "F.Cu") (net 13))
 (segment (start 35.2705 33.81) (end 35.1528 33.9277) (width 0.8) (layer "F.Cu") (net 13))
 (segment (start 26.8131 43) (end 28.9375 45.1244) (width 0.8) (layer "F.Cu") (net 13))
 (segment (start 27.9402 38) (end 23 38) (width 0.8) (layer "F.Cu") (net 13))
 (segment (start 28.9375 45.1244) (end 28.9375 45.5) (width 0.8) (layer "F.Cu") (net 13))
 (segment (start 28.9375 38.9973) (end 28.9375 40.5) (width 0.8) (layer "F.Cu") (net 13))
 (segment (start 24 43) (end 26.8131 43) (width 0.8) (layer "F.Cu") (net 13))
 (segment (start 24.9682 31.1998) (end 27.0625 29.1055) (width 0.8) (layer "F.Cu") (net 5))
 (segment (start 22.4125 22.5018) (end 17.975 26.9393) (width 0.8) (layer "F.Cu") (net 5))
 (segment (start 17.975 26.9393) (end 17.975 29.7308) (width 0.8) (layer "F.Cu") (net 5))
 (segment (start 22.4125 22) (end 22.4125 22.5018) (width 0.8) (layer "F.Cu") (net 5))
 (segment (start 27.0625 29.1055) (end 27.0625 22) (width 0.8) (layer "F.Cu") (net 5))
 (segment (start 19.444 31.1998) (end 24.9682 31.1998) (width 0.8) (layer "F.Cu") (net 5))
 (segment (start 17.975 29.7308) (end 19.444 31.1998) (width 0.8) (layer "F.Cu") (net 5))
 (segment (start 22.4125 33.35) (end 27.0625 33.35) (width 0.8) (layer "F.Cu") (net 7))
 (segment (start 27.0625 45.5) (end 22.4125 45.5) (width 0.8) (layer "F.Cu") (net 4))
 (segment (start 32 24.934784) (end 34.525216 27.46) (width 0.8) (layer "F.Cu") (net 11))
 (segment (start 13.8278 12) (end 13.6829 12) (width 0.8) (layer "F.Cu") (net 11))
 (segment (start 34.525216 27.46) (end 35.7 27.46) (width 0.8) (layer "F.Cu") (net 11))
 (segment (start 13.6829 12) (end 13.538 12) (width 0.8) (layer "F.Cu") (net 11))
 (segment (start 32 23) (end 32 24.934784) (width 0.8) (layer "F.Cu") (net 11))
 (segment (start 13.538 12) (end 11.1875 12) (width 0.8) (layer "F.Cu") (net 11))
 (segment (start 14.5875 12) (end 13.8278 12) (width 0.8) (layer "F.Cu") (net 11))
 (segment (start 2.0875 12) (end 11.1875 12) (width 0.8) (layer "F.Cu") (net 11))
 (segment (start 14 12.5875) (end 14.5875 12) (width 0.8) (layer "F.Cu") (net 11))
 (segment (start 14 15) (end 14 12.5875) (width 0.8) (layer "F.Cu") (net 11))
 (segment (start 15 16) (end 14 15) (width 0.8) (layer "F.Cu") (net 11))
 (via (at 32 23) (size 1.5) (drill 0.9) (layers "F.Cu" "B.Cu") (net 11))
 (via (at 15 16) (size 1.5) (drill 0.9) (layers "F.Cu" "B.Cu") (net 11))
 (segment (start 15 16) (end 19 16) (width 0.8) (layer "B.Cu") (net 11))
 (segment (start 19 16) (end 26 23) (width 0.8) (layer "B.Cu") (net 11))
 (segment (start 26 23) (end 32 23) (width 0.8) (layer "B.Cu") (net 11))
 (segment (start 19.7955 34.9503) (end 14.5875 29.7423) (width 0.8) (layer "F.Cu") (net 8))
 (segment (start 29.647 34.9503) (end 19.7955 34.9503) (width 0.8) (layer "F.Cu") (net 8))
 (segment (start 11.5814 26.6061) (end 12.4401 26.6061) (width 0.8) (layer "F.Cu") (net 8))
 (segment (start 14.1936 26.6061) (end 14.5875 27) (width 0.8) (layer "F.Cu") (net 8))
 (segment (start 33.9093 31.3892) (end 33.2081 31.3892) (width 0.8) (layer "F.Cu") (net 8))
 (segment (start 35.5808 31.3892) (end 35.7 31.27) (width 0.8) (layer "F.Cu") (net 8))
 (segment (start 11.1875 27) (end 11.5814 26.6061) (width 0.8) (layer "F.Cu") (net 8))
 (segment (start 33.2081 31.3892) (end 29.647 34.9503) (width 0.8) (layer "F.Cu") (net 8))
 (segment (start 14.5875 29.7423) (end 14.5875 27) (width 0.8) (layer "F.Cu") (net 8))
 (segment (start 12.4401 26.6061) (end 14.1936 26.6061) (width 0.8) (layer "F.Cu") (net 8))
 (segment (start 33.9093 31.3892) (end 35.5808 31.3892) (width 0.8) (layer "F.Cu") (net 8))
 (segment (start 30.2416 36.1741) (end 19.9035 36.1741) (width 0.8) (layer "F.Cu") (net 9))
 (segment (start 35.7 32.54) (end 34.4558 32.54) (width 0.8) (layer "F.Cu") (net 9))
 (segment (start 34.4558 32.54) (end 34.3366 32.6592) (width 0.8) (layer "F.Cu") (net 9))
 (segment (start 14.5875 41.4901) (end 14.5875 42) (width 0.8) (layer "F.Cu") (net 9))
 (segment (start 34.3366 32.6592) (end 33.7565 32.6592) (width 0.8) (layer "F.Cu") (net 9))
 (segment (start 14.5875 42) (end 11.1875 42) (width 0.8) (layer "F.Cu") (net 9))
 (segment (start 19.9035 36.1741) (end 14.5875 41.4901) (width 0.8) (layer "F.Cu") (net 9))
 (segment (start 33.7565 32.6592) (end 30.2416 36.1741) (width 0.8) (layer "F.Cu") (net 9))
 (segment (start 46.059 36.139) (end 46.059 39.2832) (width 0.8) (layer "F.Cu") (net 1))
 (segment (start 45 35.08) (end 46.059 36.139) (width 0.8) (layer "F.Cu") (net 1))
 (segment (start 30 15) (end 33.9 18.9) (width 0.8) (layer "F.Cu") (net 25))
 (segment (start 33.9 18.9) (end 34.5 18.9) (width 0.8) (layer "F.Cu") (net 25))
 (segment (start 24 15) (end 30 15) (width 0.8) (layer "F.Cu") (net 25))
 (segment (start 19.9253 26.849) (end 24 22.7743) (width 0.8) (layer "F.Cu") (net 25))
 (segment (start 19.1767 27.5976) (end 19.274 27.5003) (width 0.8) (layer "F.Cu") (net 25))
 (segment (start 22.4125 28.8651) (end 21.2795 29.9981) (width 0.8) (layer "F.Cu") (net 25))
 (segment (start 19.9418 29.9981) (end 19.1767 29.233) (width 0.8) (layer "F.Cu") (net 25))
 (segment (start 19.1767 29.233) (end 19.1767 27.5976) (width 0.8) (layer "F.Cu") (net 25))
 (segment (start 19.274 27.5003) (end 19.274 27.457734) (width 0.8) (layer "F.Cu") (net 25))
 (segment (start 19.274 27.457734) (end 19.882734 26.849) (width 0.8) (layer "F.Cu") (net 25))
 (segment (start 24 22.7743) (end 24 15) (width 0.8) (layer "F.Cu") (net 25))
 (segment (start 21.2795 29.9981) (end 19.9418 29.9981) (width 0.8) (layer "F.Cu") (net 25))
 (segment (start 19.882734 26.849) (end 19.9253 26.849) (width 0.8) (layer "F.Cu") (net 25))
 (segment (start 22.4125 28.35) (end 22.4125 28.8651) (width 0.8) (layer "F.Cu") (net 25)))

